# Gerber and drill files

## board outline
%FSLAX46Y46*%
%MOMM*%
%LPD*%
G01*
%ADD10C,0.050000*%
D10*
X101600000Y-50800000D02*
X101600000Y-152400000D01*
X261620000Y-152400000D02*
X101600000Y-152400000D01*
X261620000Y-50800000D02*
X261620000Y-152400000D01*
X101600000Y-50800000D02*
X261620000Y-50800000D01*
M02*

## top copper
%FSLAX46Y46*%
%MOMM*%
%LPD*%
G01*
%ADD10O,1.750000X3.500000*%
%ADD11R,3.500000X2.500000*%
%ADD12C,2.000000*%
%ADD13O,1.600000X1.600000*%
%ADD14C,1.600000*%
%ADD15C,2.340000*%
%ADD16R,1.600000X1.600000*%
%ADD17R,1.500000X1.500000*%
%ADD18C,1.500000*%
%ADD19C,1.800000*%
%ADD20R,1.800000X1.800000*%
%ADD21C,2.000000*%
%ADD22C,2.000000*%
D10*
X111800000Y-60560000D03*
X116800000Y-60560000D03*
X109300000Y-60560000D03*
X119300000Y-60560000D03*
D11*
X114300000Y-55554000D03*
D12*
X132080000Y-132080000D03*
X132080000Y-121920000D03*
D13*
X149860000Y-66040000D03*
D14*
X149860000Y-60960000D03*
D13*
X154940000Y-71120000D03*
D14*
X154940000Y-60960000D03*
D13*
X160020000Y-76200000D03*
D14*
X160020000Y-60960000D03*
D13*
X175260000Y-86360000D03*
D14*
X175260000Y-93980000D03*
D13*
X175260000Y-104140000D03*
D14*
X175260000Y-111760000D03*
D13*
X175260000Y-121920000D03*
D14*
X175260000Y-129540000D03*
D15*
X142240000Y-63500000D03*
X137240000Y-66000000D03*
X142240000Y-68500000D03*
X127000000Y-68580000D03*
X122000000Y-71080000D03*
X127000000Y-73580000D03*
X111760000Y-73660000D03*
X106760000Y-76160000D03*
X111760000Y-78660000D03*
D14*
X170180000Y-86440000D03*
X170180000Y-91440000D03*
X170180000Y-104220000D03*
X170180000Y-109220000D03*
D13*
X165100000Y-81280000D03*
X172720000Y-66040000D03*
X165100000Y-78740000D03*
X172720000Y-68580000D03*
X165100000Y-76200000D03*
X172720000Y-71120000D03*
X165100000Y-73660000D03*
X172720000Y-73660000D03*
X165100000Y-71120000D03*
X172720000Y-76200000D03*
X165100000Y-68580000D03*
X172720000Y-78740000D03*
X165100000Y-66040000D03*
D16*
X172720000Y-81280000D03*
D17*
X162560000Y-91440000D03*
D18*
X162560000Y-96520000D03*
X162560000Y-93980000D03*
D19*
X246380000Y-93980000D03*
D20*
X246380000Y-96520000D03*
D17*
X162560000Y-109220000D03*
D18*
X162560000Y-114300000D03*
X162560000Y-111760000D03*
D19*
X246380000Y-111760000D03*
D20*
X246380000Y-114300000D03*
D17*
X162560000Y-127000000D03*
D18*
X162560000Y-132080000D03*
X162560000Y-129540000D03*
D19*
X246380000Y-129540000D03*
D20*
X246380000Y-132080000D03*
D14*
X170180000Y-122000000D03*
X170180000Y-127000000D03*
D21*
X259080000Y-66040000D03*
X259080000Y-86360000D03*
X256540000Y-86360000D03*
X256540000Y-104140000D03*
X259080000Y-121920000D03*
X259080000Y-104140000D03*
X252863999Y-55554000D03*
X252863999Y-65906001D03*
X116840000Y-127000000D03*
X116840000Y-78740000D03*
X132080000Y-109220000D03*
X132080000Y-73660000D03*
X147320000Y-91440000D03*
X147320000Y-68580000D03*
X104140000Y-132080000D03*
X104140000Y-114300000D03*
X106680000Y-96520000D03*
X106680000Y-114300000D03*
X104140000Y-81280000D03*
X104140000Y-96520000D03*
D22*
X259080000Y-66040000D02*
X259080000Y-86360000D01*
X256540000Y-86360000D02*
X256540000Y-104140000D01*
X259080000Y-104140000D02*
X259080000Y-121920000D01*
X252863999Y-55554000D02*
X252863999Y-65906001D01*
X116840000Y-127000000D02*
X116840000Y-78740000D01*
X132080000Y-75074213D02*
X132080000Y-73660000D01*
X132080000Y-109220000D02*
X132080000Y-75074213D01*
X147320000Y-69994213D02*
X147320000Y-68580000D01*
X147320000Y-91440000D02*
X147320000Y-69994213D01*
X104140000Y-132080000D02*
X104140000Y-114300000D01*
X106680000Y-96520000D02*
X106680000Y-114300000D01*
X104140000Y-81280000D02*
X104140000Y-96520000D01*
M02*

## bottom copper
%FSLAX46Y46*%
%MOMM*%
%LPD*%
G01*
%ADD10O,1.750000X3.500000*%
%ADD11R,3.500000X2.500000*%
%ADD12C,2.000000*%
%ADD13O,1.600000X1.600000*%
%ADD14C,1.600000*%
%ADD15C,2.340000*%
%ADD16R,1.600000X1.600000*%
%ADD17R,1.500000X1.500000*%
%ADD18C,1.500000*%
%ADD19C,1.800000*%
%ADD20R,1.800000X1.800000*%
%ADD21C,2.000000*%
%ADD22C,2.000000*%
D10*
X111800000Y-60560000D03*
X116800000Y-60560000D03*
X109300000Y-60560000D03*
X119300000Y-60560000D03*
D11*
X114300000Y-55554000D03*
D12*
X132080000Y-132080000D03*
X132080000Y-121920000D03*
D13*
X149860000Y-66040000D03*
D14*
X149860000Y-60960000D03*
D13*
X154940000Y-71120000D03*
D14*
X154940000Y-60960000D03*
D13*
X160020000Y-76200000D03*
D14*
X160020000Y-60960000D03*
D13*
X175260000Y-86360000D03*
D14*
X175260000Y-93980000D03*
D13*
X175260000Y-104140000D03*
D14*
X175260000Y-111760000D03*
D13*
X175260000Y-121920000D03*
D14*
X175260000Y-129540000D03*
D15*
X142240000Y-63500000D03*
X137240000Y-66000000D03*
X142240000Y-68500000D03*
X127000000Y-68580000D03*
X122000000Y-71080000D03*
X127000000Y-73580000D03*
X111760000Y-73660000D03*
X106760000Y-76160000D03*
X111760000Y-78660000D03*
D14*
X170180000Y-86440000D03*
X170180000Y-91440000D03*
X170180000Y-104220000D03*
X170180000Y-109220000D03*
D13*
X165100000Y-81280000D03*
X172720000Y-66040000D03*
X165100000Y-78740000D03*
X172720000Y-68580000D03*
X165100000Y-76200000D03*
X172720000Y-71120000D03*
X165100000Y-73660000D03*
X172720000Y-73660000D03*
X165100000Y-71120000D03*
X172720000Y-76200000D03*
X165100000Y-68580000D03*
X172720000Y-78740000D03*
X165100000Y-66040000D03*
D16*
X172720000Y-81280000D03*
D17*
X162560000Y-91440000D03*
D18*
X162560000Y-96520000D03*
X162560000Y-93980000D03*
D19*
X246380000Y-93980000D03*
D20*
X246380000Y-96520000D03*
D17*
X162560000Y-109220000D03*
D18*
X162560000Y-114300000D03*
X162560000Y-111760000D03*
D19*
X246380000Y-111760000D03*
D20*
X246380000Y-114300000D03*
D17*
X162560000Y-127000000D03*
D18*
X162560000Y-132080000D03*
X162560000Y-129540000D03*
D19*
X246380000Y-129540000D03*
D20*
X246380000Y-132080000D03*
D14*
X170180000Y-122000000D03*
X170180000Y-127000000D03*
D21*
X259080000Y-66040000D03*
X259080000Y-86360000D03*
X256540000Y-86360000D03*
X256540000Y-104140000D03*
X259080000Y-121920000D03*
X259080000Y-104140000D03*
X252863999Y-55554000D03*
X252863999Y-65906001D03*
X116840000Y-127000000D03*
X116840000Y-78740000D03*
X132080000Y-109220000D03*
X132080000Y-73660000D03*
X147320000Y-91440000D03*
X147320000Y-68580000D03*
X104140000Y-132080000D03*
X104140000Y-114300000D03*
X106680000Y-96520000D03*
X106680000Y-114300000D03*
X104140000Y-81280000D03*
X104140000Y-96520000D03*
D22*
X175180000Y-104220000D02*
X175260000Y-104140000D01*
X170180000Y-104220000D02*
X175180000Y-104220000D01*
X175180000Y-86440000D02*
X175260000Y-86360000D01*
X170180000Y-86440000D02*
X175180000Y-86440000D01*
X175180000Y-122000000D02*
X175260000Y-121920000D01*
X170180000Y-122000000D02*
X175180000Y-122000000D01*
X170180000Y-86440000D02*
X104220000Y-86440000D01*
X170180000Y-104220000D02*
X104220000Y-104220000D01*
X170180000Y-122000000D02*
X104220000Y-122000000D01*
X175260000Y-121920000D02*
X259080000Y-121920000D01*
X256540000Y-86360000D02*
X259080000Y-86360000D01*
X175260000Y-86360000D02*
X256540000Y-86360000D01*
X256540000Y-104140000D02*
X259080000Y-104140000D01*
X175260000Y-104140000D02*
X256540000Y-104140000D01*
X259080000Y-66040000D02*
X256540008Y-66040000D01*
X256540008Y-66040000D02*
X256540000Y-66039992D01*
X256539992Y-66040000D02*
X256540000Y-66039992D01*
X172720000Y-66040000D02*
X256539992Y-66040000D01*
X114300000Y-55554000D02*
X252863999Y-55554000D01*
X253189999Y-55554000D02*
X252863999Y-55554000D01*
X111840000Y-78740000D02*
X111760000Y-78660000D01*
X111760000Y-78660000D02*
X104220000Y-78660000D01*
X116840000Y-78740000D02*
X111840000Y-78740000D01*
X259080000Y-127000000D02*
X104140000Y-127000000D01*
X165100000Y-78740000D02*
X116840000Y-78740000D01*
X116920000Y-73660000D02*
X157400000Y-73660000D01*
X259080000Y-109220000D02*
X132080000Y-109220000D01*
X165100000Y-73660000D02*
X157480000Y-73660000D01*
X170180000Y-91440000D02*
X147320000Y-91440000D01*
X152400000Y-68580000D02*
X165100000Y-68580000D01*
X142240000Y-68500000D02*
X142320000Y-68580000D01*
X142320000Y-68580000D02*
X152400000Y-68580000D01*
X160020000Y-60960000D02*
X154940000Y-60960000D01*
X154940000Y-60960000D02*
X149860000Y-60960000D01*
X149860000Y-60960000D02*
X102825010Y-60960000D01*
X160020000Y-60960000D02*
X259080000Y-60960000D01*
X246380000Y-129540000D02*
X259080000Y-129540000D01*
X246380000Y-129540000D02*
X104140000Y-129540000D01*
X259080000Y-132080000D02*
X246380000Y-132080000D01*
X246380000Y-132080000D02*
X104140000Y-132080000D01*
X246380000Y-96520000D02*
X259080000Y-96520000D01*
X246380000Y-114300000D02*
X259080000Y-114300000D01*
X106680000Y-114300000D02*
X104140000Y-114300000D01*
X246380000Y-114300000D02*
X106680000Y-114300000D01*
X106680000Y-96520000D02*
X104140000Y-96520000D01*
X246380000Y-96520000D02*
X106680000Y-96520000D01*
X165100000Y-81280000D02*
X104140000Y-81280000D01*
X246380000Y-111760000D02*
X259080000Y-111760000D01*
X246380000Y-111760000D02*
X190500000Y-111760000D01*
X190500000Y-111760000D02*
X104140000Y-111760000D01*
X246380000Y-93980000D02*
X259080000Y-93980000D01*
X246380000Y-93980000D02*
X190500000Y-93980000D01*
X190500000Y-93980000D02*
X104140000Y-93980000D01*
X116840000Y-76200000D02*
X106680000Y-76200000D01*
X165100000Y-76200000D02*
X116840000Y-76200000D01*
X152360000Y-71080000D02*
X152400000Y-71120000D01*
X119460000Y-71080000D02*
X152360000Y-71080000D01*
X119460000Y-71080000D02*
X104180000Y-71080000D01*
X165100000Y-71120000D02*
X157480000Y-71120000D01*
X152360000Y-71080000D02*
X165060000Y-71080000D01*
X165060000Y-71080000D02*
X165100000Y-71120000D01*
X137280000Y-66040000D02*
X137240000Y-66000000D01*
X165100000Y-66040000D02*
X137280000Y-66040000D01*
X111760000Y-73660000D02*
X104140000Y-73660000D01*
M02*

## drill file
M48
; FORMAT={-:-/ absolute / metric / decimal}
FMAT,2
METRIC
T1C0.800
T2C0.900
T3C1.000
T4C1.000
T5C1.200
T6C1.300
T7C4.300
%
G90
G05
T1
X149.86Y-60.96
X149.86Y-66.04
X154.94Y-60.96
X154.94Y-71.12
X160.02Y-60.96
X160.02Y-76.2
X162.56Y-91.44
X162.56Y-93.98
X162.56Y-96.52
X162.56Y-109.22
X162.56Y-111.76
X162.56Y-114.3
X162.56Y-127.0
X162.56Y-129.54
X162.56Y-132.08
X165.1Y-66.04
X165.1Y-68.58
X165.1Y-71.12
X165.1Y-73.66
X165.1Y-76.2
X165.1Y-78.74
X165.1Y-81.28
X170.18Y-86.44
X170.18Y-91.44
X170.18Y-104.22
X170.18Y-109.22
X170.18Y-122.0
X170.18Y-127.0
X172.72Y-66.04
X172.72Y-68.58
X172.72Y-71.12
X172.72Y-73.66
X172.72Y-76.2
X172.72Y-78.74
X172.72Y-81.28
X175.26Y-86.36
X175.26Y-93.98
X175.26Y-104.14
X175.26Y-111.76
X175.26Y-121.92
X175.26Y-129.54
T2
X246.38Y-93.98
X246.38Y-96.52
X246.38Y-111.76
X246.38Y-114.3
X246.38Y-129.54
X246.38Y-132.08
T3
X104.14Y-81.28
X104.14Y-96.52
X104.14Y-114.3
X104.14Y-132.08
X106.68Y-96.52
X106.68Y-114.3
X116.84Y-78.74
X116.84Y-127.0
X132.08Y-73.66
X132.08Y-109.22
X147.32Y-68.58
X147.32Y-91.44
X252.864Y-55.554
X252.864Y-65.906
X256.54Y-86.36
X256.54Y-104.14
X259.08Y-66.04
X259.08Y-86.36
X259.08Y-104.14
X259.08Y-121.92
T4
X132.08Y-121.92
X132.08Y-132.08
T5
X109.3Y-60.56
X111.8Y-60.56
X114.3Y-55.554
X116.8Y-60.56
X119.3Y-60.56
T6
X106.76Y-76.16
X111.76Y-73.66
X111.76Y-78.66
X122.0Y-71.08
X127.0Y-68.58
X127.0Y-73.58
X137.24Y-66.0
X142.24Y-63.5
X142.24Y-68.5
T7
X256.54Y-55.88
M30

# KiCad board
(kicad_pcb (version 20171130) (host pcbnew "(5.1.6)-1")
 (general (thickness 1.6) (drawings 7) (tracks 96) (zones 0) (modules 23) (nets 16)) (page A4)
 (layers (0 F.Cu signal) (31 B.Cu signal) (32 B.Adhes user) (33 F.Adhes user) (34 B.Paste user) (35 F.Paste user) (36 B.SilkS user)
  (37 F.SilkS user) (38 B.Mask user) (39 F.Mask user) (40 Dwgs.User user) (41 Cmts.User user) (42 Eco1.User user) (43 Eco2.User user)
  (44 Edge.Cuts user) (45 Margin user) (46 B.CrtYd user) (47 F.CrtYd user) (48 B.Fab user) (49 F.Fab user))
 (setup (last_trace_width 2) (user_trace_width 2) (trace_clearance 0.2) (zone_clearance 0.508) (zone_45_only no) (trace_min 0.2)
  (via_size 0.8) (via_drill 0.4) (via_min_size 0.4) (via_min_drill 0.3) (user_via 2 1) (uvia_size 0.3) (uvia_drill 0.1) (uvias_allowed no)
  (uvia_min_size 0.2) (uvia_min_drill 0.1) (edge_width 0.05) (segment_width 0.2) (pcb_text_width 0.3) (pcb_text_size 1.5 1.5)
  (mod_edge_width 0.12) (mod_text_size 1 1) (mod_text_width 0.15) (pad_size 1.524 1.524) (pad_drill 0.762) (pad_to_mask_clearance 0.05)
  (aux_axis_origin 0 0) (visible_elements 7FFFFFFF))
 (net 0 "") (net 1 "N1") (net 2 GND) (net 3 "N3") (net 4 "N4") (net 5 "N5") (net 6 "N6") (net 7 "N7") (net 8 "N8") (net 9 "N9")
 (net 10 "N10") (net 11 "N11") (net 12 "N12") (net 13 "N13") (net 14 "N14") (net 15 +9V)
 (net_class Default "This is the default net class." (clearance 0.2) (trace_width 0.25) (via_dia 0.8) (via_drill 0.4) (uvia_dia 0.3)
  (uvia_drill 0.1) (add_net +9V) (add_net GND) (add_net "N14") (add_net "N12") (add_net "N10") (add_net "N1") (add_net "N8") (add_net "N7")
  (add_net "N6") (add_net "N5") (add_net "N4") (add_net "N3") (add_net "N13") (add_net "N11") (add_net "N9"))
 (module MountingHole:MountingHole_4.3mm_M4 (layer F.Cu) (at 256.54 55.88)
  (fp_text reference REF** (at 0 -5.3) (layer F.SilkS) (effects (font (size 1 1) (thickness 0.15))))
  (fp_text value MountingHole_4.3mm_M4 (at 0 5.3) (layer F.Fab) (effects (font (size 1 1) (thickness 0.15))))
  (pad 1 np_thru_hole circle (at 0 0) (size 4.3 4.3) (drill 4.3) (layers *.Cu *.Mask)))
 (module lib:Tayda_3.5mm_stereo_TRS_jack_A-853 (layer F.Cu) (at 114.3 57.15)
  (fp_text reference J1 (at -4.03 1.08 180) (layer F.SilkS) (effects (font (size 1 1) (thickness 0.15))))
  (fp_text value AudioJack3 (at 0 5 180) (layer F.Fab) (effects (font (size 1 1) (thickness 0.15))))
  (pad 5 thru_hole oval (at -2.5 3.41) (size 1.75 3.5) (drill 1.2) (layers *.Cu *.Mask F.SilkS) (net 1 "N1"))
  (pad 4 thru_hole oval (at 2.5 3.41) (size 1.75 3.5) (drill 1.2) (layers *.Cu *.Mask F.SilkS) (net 1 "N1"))
  (pad 3 thru_hole oval (at -5 3.41) (size 1.75 3.5) (drill 1.2) (layers *.Cu *.Mask F.SilkS) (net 1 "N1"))
  (pad 2 thru_hole oval (at 5 3.41) (size 1.75 3.5) (drill 1.2) (layers *.Cu *.Mask F.SilkS) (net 1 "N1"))
  (pad 1 thru_hole rect (at 0 -1.596) (size 3.5 2.5) (drill 1.2) (layers *.Cu *.Mask F.SilkS) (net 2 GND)))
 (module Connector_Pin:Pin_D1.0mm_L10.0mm (layer F.Cu) (at 132.08 132.08)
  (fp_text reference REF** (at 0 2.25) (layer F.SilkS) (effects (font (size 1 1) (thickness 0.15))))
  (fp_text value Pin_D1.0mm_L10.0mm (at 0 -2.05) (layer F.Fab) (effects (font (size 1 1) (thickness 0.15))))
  (pad 1 thru_hole circle (at 0 0) (size 2 2) (drill 1) (layers *.Cu *.Mask)))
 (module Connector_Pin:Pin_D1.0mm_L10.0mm (layer F.Cu) (at 132.08 121.92)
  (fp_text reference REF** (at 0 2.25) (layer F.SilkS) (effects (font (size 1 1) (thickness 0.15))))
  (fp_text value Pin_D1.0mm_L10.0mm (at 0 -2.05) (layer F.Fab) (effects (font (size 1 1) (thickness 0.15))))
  (pad 1 thru_hole circle (at 0 0) (size 2 2) (drill 1) (layers *.Cu *.Mask)))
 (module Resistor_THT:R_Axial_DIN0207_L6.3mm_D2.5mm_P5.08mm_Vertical (layer F.Cu) (at 149.86 60.96 270)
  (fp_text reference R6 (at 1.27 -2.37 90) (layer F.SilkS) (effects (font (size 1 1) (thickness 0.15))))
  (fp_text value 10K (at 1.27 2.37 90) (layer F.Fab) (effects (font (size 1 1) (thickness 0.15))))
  (pad 2 thru_hole oval (at 5.08 0 270) (size 1.6 1.6) (drill 0.8) (layers *.Cu *.Mask) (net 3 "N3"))
  (pad 1 thru_hole circle (at 0 0 270) (size 1.6 1.6) (drill 0.8) (layers *.Cu *.Mask) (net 1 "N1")))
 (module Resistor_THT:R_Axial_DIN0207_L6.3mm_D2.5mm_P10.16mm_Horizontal (layer F.Cu) (at 154.94 60.96 270)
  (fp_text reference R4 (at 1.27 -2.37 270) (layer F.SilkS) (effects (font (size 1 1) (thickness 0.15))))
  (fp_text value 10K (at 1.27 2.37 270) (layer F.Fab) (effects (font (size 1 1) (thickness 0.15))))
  (pad 2 thru_hole oval (at 10.16 0 270) (size 1.6 1.6) (drill 0.8) (layers *.Cu *.Mask) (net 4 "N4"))
  (pad 1 thru_hole circle (at 0 0 270) (size 1.6 1.6) (drill 0.8) (layers *.Cu *.Mask) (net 1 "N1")))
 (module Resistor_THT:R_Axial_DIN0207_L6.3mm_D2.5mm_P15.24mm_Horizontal (layer F.Cu) (at 160.02 60.96 270)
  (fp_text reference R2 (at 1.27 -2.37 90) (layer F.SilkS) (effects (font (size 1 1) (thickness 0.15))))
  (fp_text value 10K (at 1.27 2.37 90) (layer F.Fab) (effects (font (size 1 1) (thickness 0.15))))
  (pad 2 thru_hole oval (at 15.24 0 270) (size 1.6 1.6) (drill 0.8) (layers *.Cu *.Mask) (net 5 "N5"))
  (pad 1 thru_hole circle (at 0 0 270) (size 1.6 1.6) (drill 0.8) (layers *.Cu *.Mask) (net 1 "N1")))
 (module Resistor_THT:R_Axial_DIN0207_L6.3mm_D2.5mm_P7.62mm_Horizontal (layer F.Cu) (at 175.26 93.98 90)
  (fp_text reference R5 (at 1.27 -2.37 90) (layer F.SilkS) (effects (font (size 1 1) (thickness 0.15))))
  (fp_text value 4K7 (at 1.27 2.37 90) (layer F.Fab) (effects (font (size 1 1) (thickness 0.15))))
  (pad 2 thru_hole oval (at 7.62 0 90) (size 1.6 1.6) (drill 0.8) (layers *.Cu *.Mask) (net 2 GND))
  (pad 1 thru_hole circle (at 0 0 90) (size 1.6 1.6) (drill 0.8) (layers *.Cu *.Mask) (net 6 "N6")))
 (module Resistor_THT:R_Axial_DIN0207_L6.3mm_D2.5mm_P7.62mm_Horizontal (layer F.Cu) (at 175.26 111.76 90)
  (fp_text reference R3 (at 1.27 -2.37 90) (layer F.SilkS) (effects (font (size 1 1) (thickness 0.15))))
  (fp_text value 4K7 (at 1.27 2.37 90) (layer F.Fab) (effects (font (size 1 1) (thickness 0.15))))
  (pad 2 thru_hole oval (at 7.62 0 90) (size 1.6 1.6) (drill 0.8) (layers *.Cu *.Mask) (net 2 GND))
  (pad 1 thru_hole circle (at 0 0 90) (size 1.6 1.6) (drill 0.8) (layers *.Cu *.Mask) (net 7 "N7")))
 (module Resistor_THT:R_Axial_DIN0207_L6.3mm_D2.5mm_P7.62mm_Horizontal (layer F.Cu) (at 175.26 129.54 90)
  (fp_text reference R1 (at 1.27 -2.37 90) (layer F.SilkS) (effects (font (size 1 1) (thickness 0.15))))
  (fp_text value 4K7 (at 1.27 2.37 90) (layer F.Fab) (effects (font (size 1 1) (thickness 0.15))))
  (pad 2 thru_hole oval (at 7.62 0 90) (size 1.6 1.6) (drill 0.8) (layers *.Cu *.Mask) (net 2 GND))
  (pad 1 thru_hole circle (at 0 0 90) (size 1.6 1.6) (drill 0.8) (layers *.Cu *.Mask) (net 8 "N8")))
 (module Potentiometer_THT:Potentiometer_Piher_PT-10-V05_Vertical (layer F.Cu) (at 142.24 63.5 180)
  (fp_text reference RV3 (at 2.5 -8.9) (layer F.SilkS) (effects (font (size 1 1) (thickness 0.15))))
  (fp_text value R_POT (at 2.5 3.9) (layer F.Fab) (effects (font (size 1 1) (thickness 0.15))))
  (pad 1 thru_hole circle (at 0 0 180) (size 2.34 2.34) (drill 1.3) (layers *.Cu *.Mask) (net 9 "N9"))
  (pad 2 thru_hole circle (at 5 -2.5 180) (size 2.34 2.34) (drill 1.3) (layers *.Cu *.Mask) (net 3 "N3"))
  (pad 3 thru_hole circle (at 0 -5 180) (size 2.34 2.34) (drill 1.3) (layers *.Cu *.Mask) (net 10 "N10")))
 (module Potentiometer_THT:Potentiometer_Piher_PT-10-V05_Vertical (layer F.Cu) (at 127 68.58 180)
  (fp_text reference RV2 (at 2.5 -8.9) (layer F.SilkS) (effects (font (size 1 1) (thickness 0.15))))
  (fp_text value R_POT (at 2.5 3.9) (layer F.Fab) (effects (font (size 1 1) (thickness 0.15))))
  (pad 1 thru_hole circle (at 0 0 180) (size 2.34 2.34) (drill 1.3) (layers *.Cu *.Mask) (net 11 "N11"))
  (pad 2 thru_hole circle (at 5 -2.5 180) (size 2.34 2.34) (drill 1.3) (layers *.Cu *.Mask) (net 4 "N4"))
  (pad 3 thru_hole circle (at 0 -5 180) (size 2.34 2.34) (drill 1.3) (layers *.Cu *.Mask) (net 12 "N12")))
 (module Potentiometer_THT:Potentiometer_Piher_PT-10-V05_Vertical (layer F.Cu) (at 111.76 73.66 180)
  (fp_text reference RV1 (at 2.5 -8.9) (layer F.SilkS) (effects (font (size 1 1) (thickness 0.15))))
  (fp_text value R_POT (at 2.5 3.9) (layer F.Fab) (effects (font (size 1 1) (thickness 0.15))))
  (pad 1 thru_hole circle (at 0 0 180) (size 2.34 2.34) (drill 1.3) (layers *.Cu *.Mask) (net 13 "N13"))
  (pad 2 thru_hole circle (at 5 -2.5 180) (size 2.34 2.34) (drill 1.3) (layers *.Cu *.Mask) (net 5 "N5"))
  (pad 3 thru_hole circle (at 0 -5 180) (size 2.34 2.34) (drill 1.3) (layers *.Cu *.Mask) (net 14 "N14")))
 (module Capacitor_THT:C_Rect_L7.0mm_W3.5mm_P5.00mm (layer F.Cu) (at 170.18 91.44 90)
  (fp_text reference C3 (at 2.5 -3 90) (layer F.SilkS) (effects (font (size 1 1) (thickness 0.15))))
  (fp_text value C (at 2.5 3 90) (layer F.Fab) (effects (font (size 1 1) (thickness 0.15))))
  (pad 2 thru_hole circle (at 5 0 90) (size 1.6 1.6) (drill 0.8) (layers *.Cu *.Mask) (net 2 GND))
  (pad 1 thru_hole circle (at 0 0 90) (size 1.6 1.6) (drill 0.8) (layers *.Cu *.Mask) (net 10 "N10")))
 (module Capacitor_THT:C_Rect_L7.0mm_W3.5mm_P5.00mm (layer F.Cu) (at 170.18 109.22 90)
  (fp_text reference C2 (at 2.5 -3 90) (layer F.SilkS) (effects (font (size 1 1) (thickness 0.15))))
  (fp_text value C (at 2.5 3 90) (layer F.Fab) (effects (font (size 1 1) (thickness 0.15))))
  (pad 2 thru_hole circle (at 5 0 90) (size 1.6 1.6) (drill 0.8) (layers *.Cu *.Mask) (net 2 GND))
  (pad 1 thru_hole circle (at 0 0 90) (size 1.6 1.6) (drill 0.8) (layers *.Cu *.Mask) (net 12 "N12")))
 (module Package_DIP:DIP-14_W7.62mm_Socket (layer F.Cu) (at 172.72 81.28 180)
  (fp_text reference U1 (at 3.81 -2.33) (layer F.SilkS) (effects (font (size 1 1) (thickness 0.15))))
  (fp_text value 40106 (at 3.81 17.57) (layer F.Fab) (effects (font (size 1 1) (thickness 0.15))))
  (pad 14 thru_hole oval (at 7.62 0 180) (size 1.6 1.6) (drill 0.8) (layers *.Cu *.Mask) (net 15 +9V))
  (pad 7 thru_hole oval (at 0 15.24 180) (size 1.6 1.6) (drill 0.8) (layers *.Cu *.Mask) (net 2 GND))
  (pad 13 thru_hole oval (at 7.62 2.54 180) (size 1.6 1.6) (drill 0.8) (layers *.Cu *.Mask) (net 14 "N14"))
  (pad 6 thru_hole oval (at 0 12.7 180) (size 1.6 1.6) (drill 0.8) (layers *.Cu *.Mask))
  (pad 12 thru_hole oval (at 7.62 5.08 180) (size 1.6 1.6) (drill 0.8) (layers *.Cu *.Mask) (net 5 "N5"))
  (pad 5 thru_hole oval (at 0 10.16 180) (size 1.6 1.6) (drill 0.8) (layers *.Cu *.Mask))
  (pad 11 thru_hole oval (at 7.62 7.62 180) (size 1.6 1.6) (drill 0.8) (layers *.Cu *.Mask) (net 12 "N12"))
  (pad 4 thru_hole oval (at 0 7.62 180) (size 1.6 1.6) (drill 0.8) (layers *.Cu *.Mask))
  (pad 10 thru_hole oval (at 7.62 10.16 180) (size 1.6 1.6) (drill 0.8) (layers *.Cu *.Mask) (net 4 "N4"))
  (pad 3 thru_hole oval (at 0 5.08 180) (size 1.6 1.6) (drill 0.8) (layers *.Cu *.Mask))
  (pad 9 thru_hole oval (at 7.62 12.7 180) (size 1.6 1.6) (drill 0.8) (layers *.Cu *.Mask) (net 10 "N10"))
  (pad 2 thru_hole oval (at 0 2.54 180) (size 1.6 1.6) (drill 0.8) (layers *.Cu *.Mask))
  (pad 8 thru_hole oval (at 7.62 15.24 180) (size 1.6 1.6) (drill 0.8) (layers *.Cu *.Mask) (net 3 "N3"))
  (pad 1 thru_hole rect (at 0 0 180) (size 1.6 1.6) (drill 0.8) (layers *.Cu *.Mask)))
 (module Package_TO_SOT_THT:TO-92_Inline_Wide (layer F.Cu) (at 162.56 91.44 270)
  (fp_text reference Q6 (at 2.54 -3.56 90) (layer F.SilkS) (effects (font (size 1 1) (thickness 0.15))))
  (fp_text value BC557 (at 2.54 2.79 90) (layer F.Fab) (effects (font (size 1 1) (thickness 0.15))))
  (pad 1 thru_hole rect (at 0 0) (size 1.5 1.5) (drill 0.8) (layers *.Cu *.Mask) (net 10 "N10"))
  (pad 3 thru_hole circle (at 5.08 0) (size 1.5 1.5) (drill 0.8) (layers *.Cu *.Mask) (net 15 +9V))
  (pad 2 thru_hole circle (at 2.54 0) (size 1.5 1.5) (drill 0.8) (layers *.Cu *.Mask) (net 6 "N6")))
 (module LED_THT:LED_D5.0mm (layer F.Cu) (at 246.38 96.52 90)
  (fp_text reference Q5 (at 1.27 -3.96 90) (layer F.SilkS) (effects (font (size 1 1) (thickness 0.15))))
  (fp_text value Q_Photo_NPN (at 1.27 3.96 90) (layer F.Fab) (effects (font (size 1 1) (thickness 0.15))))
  (pad 2 thru_hole circle (at 2.54 0 90) (size 1.8 1.8) (drill 0.9) (layers *.Cu *.Mask) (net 6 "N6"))
  (pad 1 thru_hole rect (at 0 0 90) (size 1.8 1.8) (drill 0.9) (layers *.Cu *.Mask) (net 15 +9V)))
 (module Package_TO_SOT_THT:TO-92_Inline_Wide (layer F.Cu) (at 162.56 109.22 270)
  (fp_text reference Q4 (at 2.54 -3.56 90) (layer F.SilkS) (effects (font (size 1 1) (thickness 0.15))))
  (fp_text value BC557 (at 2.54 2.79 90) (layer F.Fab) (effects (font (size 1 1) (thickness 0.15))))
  (pad 1 thru_hole rect (at 0 0) (size 1.5 1.5) (drill 0.8) (layers *.Cu *.Mask) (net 12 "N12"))
  (pad 3 thru_hole circle (at 5.08 0) (size 1.5 1.5) (drill 0.8) (layers *.Cu *.Mask) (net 15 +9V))
  (pad 2 thru_hole circle (at 2.54 0) (size 1.5 1.5) (drill 0.8) (layers *.Cu *.Mask) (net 7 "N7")))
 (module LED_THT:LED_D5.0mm (layer F.Cu) (at 246.38 114.3 90)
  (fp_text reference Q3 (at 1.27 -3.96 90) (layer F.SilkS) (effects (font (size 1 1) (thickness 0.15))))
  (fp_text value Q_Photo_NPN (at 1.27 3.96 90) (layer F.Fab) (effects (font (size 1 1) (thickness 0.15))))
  (pad 2 thru_hole circle (at 2.54 0 90) (size 1.8 1.8) (drill 0.9) (layers *.Cu *.Mask) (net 7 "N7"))
  (pad 1 thru_hole rect (at 0 0 90) (size 1.8 1.8) (drill 0.9) (layers *.Cu *.Mask) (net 15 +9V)))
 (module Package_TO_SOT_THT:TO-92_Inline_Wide (layer F.Cu) (at 162.56 127 270)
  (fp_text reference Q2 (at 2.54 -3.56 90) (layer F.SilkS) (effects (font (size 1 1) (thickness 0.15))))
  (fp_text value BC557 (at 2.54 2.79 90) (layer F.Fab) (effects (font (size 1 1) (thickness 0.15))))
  (pad 1 thru_hole rect (at 0 0) (size 1.5 1.5) (drill 0.8) (layers *.Cu *.Mask) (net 14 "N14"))
  (pad 3 thru_hole circle (at 5.08 0) (size 1.5 1.5) (drill 0.8) (layers *.Cu *.Mask) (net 15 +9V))
  (pad 2 thru_hole circle (at 2.54 0) (size 1.5 1.5) (drill 0.8) (layers *.Cu *.Mask) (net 8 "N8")))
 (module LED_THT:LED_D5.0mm (layer F.Cu) (at 246.38 132.08 90)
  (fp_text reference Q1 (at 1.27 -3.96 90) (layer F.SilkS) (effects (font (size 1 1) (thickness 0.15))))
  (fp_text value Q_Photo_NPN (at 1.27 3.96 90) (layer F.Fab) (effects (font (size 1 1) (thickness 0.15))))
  (pad 2 thru_hole circle (at 2.54 0 90) (size 1.8 1.8) (drill 0.9) (layers *.Cu *.Mask) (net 8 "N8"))
  (pad 1 thru_hole rect (at 0 0 90) (size 1.8 1.8) (drill 0.9) (layers *.Cu *.Mask) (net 15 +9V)))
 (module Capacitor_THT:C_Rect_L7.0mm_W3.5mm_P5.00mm (layer F.Cu) (at 170.18 127 90)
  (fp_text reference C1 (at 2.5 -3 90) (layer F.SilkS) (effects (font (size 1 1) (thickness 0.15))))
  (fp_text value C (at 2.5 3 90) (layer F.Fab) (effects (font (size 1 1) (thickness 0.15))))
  (pad 2 thru_hole circle (at 5 0 90) (size 1.6 1.6) (drill 0.8) (layers *.Cu *.Mask) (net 2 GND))
  (pad 1 thru_hole circle (at 0 0 90) (size 1.6 1.6) (drill 0.8) (layers *.Cu *.Mask) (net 14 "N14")))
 (gr_line (start 101.6 50.8) (end 101.6 152.4) (layer Edge.Cuts) (width 0.05))
 (gr_line (start 261.62 152.4) (end 101.6 152.4) (layer Edge.Cuts) (width 0.05))
 (gr_line (start 261.62 50.8) (end 261.62 152.4) (layer Edge.Cuts) (width 0.05))
 (gr_line (start 101.6 50.8) (end 261.62 50.8) (layer Edge.Cuts) (width 0.05))
 (segment (start 175.18 104.22) (end 175.26 104.14) (width 2) (layer B.Cu) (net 2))
 (segment (start 170.18 104.22) (end 175.18 104.22) (width 2) (layer B.Cu) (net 2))
 (segment (start 175.18 86.44) (end 175.26 86.36) (width 2) (layer B.Cu) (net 2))
 (segment (start 170.18 86.44) (end 175.18 86.44) (width 2) (layer B.Cu) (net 2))
 (segment (start 175.18 122) (end 175.26 121.92) (width 2) (layer B.Cu) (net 2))
 (segment (start 170.18 122) (end 175.18 122) (width 2) (layer B.Cu) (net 2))
 (segment (start 170.18 86.44) (end 104.22 86.44) (width 2) (layer B.Cu) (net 2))
 (segment (start 170.18 104.22) (end 104.22 104.22) (width 2) (layer B.Cu) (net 2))
 (segment (start 170.18 122) (end 104.22 122) (width 2) (layer B.Cu) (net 2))
 (segment (start 175.26 121.92) (end 259.08 121.92) (width 2) (layer B.Cu) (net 2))
 (via (at 259.08 66.04) (size 2) (drill 1) (layers F.Cu B.Cu) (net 2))
 (via (at 259.08 86.36) (size 2) (drill 1) (layers F.Cu B.Cu) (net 2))
 (segment (start 259.08 66.04) (end 259.08 86.36) (width 2) (layer F.Cu) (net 2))
 (via (at 256.54 86.36) (size 2) (drill 1) (layers F.Cu B.Cu) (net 2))
 (segment (start 256.54 86.36) (end 259.08 86.36) (width 2) (layer B.Cu) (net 2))
 (segment (start 175.26 86.36) (end 256.54 86.36) (width 2) (layer B.Cu) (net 2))
 (via (at 256.54 104.14) (size 2) (drill 1) (layers F.Cu B.Cu) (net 2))
 (segment (start 256.54 104.14) (end 259.08 104.14) (width 2) (layer B.Cu) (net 2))
 (segment (start 175.26 104.14) (end 256.54 104.14) (width 2) (layer B.Cu) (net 2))
 (via (at 259.08 121.92) (size 2) (drill 1) (layers F.Cu B.Cu) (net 2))
 (via (at 259.08 104.14) (size 2) (drill 1) (layers F.Cu B.Cu) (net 2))
 (segment (start 256.54 86.36) (end 256.54 104.14) (width 2) (layer F.Cu) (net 2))
 (segment (start 259.08 104.14) (end 259.08 121.92) (width 2) (layer F.Cu) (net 2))
 (segment (start 259.08 66.04) (end 256.540008 66.04) (width 2) (layer B.Cu) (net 2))
 (segment (start 256.540008 66.04) (end 256.54 66.039992) (width 2) (layer B.Cu) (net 2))
 (segment (start 256.539992 66.04) (end 256.54 66.039992) (width 2) (layer B.Cu) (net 2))
 (segment (start 172.72 66.04) (end 256.539992 66.04) (width 2) (layer B.Cu) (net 2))
 (segment (start 114.3 55.554) (end 252.863999 55.554) (width 2) (layer B.Cu) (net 2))
 (via (at 252.863999 55.554) (size 2) (drill 1) (layers F.Cu B.Cu) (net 2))
 (segment (start 253.189999 55.554) (end 252.863999 55.554) (width 2) (layer B.Cu) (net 2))
 (segment (start 252.863999 55.554) (end 252.863999 65.906001) (width 2) (layer F.Cu) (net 2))
 (via (at 252.863999 65.906001) (size 2) (drill 1) (layers F.Cu B.Cu) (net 2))
 (segment (start 111.84 78.74) (end 111.76 78.66) (width 2) (layer B.Cu) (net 14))
 (segment (start 111.76 78.66) (end 104.22 78.66) (width 2) (layer B.Cu) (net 14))
 (segment (start 116.84 78.74) (end 111.84 78.74) (width 2) (layer B.Cu) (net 14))
 (via (at 116.84 127) (size 2) (drill 1) (layers F.Cu B.Cu) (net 14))
 (segment (start 116.84 127) (end 116.84 78.74) (width 2) (layer F.Cu) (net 14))
 (via (at 116.84 78.74) (size 2) (drill 1) (layers F.Cu B.Cu) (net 14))
 (segment (start 259.08 127) (end 104.14 127) (width 2) (layer B.Cu) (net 14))
 (segment (start 165.1 78.74) (end 116.84 78.74) (width 2) (layer B.Cu) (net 14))
 (via (at 132.08 109.22) (size 2) (drill 1) (layers F.Cu B.Cu) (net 12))
 (via (at 132.08 73.66) (size 2) (drill 1) (layers F.Cu B.Cu) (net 12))
 (segment (start 116.92 73.66) (end 157.4 73.66) (width 2) (layer B.Cu) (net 12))
 (segment (start 132.08 75.074213) (end 132.08 73.66) (width 2) (layer F.Cu) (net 12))
 (segment (start 132.08 109.22) (end 132.08 75.074213) (width 2) (layer F.Cu) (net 12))
 (segment (start 259.08 109.22) (end 132.08 109.22) (width 2) (layer B.Cu) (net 12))
 (segment (start 165.1 73.66) (end 157.48 73.66) (width 2) (layer B.Cu) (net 12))
 (via (at 147.32 91.44) (size 2) (drill 1) (layers F.Cu B.Cu) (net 10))
 (via (at 147.32 68.58) (size 2) (drill 1) (layers F.Cu B.Cu) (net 10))
 (segment (start 147.32 69.994213) (end 147.32 68.58) (width 2) (layer F.Cu) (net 10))
 (segment (start 147.32 91.44) (end 147.32 69.994213) (width 2) (layer F.Cu) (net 10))
 (segment (start 170.18 91.44) (end 147.32 91.44) (width 2) (layer B.Cu) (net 10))
 (segment (start 152.4 68.58) (end 165.1 68.58) (width 2) (layer B.Cu) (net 10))
 (segment (start 142.24 68.5) (end 142.32 68.58) (width 2) (layer B.Cu) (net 10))
 (segment (start 142.32 68.58) (end 152.4 68.58) (width 2) (layer B.Cu) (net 10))
 (segment (start 160.02 60.96) (end 154.94 60.96) (width 2) (layer B.Cu) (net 1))
 (segment (start 154.94 60.96) (end 149.86 60.96) (width 2) (layer B.Cu) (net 1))
 (segment (start 149.86 60.96) (end 102.82501 60.96) (width 2) (layer B.Cu) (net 1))
 (segment (start 160.02 60.96) (end 259.08 60.96) (width 2) (layer B.Cu) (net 1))
 (segment (start 246.38 129.54) (end 259.08 129.54) (width 2) (layer B.Cu) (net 8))
 (segment (start 246.38 129.54) (end 104.14 129.54) (width 2) (layer B.Cu) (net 8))
 (segment (start 259.08 132.08) (end 246.38 132.08) (width 2) (layer B.Cu) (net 15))
 (segment (start 246.38 132.08) (end 104.14 132.08) (width 2) (layer B.Cu) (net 15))
 (segment (start 246.38 96.52) (end 259.08 96.52) (width 2) (layer B.Cu) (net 15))
 (segment (start 246.38 114.3) (end 259.08 114.3) (width 2) (layer B.Cu) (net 15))
 (via (at 104.14 132.08) (size 2) (drill 1) (layers F.Cu B.Cu) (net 15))
 (via (at 104.14 114.3) (size 2) (drill 1) (layers F.Cu B.Cu) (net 15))
 (segment (start 104.14 132.08) (end 104.14 114.3) (width 2) (layer F.Cu) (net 15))
 (segment (start 106.68 114.3) (end 104.14 114.3) (width 2) (layer B.Cu) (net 15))
 (segment (start 246.38 114.3) (end 106.68 114.3) (width 2) (layer B.Cu) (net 15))
 (via (at 106.68 96.52) (size 2) (drill 1) (layers F.Cu B.Cu) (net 15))
 (segment (start 106.68 96.52) (end 104.14 96.52) (width 2) (layer B.Cu) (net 15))
 (segment (start 246.38 96.52) (end 106.68 96.52) (width 2) (layer B.Cu) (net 15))
 (segment (start 106.68 96.52) (end 106.68 114.3) (width 2) (layer F.Cu) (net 15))
 (via (at 106.68 114.3) (size 2) (drill 1) (layers F.Cu B.Cu) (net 15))
 (via (at 104.14 81.28) (size 2) (drill 1) (layers F.Cu B.Cu) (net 15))
 (via (at 104.14 96.52) (size 2) (drill 1) (layers F.Cu B.Cu) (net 15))
 (segment (start 104.14 81.28) (end 104.14 96.52) (width 2) (layer F.Cu) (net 15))
 (segment (start 165.1 81.28) (end 104.14 81.28) (width 2) (layer B.Cu) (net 15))
 (segment (start 246.38 111.76) (end 259.08 111.76) (width 2) (layer B.Cu) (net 7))
 (segment (start 246.38 111.76) (end 190.5 111.76) (width 2) (layer B.Cu) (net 7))
 (segment (start 190.5 111.76) (end 104.14 111.76) (width 2) (layer B.Cu) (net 7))
 (segment (start 246.38 93.98) (end 259.08 93.98) (width 2) (layer B.Cu) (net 6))
 (segment (start 246.38 93.98) (end 190.5 93.98) (width 2) (layer B.Cu) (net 6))
 (segment (start 190.5 93.98) (end 104.14 93.98) (width 2) (layer B.Cu) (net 6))
 (segment (start 116.84 76.2) (end 106.68 76.2) (width 2) (layer B.Cu) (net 5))
 (segment (start 165.1 76.2) (end 116.84 76.2) (width 2) (layer B.Cu) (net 5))
 (segment (start 152.36 71.08) (end 152.4 71.12) (width 2) (layer B.Cu) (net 4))
 (segment (start 119.46 71.08) (end 152.36 71.08) (width 2) (layer B.Cu) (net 4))
 (segment (start 119.46 71.08) (end 104.18 71.08) (width 2) (layer B.Cu) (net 4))
 (segment (start 165.1 71.12) (end 157.48 71.12) (width 2) (layer B.Cu) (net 4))
 (segment (start 152.36 71.08) (end 165.06 71.08) (width 2) (layer B.Cu) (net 4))
 (segment (start 165.06 71.08) (end 165.1 71.12) (width 2) (layer B.Cu) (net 4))
 (segment (start 137.28 66.04) (end 137.24 66) (width 2) (layer B.Cu) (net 3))
 (segment (start 165.1 66.04) (end 137.28 66.04) (width 2) (layer B.Cu) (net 3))
 (segment (start 111.76 73.66) (end 104.14 73.66) (width 2) (layer B.Cu) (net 13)))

